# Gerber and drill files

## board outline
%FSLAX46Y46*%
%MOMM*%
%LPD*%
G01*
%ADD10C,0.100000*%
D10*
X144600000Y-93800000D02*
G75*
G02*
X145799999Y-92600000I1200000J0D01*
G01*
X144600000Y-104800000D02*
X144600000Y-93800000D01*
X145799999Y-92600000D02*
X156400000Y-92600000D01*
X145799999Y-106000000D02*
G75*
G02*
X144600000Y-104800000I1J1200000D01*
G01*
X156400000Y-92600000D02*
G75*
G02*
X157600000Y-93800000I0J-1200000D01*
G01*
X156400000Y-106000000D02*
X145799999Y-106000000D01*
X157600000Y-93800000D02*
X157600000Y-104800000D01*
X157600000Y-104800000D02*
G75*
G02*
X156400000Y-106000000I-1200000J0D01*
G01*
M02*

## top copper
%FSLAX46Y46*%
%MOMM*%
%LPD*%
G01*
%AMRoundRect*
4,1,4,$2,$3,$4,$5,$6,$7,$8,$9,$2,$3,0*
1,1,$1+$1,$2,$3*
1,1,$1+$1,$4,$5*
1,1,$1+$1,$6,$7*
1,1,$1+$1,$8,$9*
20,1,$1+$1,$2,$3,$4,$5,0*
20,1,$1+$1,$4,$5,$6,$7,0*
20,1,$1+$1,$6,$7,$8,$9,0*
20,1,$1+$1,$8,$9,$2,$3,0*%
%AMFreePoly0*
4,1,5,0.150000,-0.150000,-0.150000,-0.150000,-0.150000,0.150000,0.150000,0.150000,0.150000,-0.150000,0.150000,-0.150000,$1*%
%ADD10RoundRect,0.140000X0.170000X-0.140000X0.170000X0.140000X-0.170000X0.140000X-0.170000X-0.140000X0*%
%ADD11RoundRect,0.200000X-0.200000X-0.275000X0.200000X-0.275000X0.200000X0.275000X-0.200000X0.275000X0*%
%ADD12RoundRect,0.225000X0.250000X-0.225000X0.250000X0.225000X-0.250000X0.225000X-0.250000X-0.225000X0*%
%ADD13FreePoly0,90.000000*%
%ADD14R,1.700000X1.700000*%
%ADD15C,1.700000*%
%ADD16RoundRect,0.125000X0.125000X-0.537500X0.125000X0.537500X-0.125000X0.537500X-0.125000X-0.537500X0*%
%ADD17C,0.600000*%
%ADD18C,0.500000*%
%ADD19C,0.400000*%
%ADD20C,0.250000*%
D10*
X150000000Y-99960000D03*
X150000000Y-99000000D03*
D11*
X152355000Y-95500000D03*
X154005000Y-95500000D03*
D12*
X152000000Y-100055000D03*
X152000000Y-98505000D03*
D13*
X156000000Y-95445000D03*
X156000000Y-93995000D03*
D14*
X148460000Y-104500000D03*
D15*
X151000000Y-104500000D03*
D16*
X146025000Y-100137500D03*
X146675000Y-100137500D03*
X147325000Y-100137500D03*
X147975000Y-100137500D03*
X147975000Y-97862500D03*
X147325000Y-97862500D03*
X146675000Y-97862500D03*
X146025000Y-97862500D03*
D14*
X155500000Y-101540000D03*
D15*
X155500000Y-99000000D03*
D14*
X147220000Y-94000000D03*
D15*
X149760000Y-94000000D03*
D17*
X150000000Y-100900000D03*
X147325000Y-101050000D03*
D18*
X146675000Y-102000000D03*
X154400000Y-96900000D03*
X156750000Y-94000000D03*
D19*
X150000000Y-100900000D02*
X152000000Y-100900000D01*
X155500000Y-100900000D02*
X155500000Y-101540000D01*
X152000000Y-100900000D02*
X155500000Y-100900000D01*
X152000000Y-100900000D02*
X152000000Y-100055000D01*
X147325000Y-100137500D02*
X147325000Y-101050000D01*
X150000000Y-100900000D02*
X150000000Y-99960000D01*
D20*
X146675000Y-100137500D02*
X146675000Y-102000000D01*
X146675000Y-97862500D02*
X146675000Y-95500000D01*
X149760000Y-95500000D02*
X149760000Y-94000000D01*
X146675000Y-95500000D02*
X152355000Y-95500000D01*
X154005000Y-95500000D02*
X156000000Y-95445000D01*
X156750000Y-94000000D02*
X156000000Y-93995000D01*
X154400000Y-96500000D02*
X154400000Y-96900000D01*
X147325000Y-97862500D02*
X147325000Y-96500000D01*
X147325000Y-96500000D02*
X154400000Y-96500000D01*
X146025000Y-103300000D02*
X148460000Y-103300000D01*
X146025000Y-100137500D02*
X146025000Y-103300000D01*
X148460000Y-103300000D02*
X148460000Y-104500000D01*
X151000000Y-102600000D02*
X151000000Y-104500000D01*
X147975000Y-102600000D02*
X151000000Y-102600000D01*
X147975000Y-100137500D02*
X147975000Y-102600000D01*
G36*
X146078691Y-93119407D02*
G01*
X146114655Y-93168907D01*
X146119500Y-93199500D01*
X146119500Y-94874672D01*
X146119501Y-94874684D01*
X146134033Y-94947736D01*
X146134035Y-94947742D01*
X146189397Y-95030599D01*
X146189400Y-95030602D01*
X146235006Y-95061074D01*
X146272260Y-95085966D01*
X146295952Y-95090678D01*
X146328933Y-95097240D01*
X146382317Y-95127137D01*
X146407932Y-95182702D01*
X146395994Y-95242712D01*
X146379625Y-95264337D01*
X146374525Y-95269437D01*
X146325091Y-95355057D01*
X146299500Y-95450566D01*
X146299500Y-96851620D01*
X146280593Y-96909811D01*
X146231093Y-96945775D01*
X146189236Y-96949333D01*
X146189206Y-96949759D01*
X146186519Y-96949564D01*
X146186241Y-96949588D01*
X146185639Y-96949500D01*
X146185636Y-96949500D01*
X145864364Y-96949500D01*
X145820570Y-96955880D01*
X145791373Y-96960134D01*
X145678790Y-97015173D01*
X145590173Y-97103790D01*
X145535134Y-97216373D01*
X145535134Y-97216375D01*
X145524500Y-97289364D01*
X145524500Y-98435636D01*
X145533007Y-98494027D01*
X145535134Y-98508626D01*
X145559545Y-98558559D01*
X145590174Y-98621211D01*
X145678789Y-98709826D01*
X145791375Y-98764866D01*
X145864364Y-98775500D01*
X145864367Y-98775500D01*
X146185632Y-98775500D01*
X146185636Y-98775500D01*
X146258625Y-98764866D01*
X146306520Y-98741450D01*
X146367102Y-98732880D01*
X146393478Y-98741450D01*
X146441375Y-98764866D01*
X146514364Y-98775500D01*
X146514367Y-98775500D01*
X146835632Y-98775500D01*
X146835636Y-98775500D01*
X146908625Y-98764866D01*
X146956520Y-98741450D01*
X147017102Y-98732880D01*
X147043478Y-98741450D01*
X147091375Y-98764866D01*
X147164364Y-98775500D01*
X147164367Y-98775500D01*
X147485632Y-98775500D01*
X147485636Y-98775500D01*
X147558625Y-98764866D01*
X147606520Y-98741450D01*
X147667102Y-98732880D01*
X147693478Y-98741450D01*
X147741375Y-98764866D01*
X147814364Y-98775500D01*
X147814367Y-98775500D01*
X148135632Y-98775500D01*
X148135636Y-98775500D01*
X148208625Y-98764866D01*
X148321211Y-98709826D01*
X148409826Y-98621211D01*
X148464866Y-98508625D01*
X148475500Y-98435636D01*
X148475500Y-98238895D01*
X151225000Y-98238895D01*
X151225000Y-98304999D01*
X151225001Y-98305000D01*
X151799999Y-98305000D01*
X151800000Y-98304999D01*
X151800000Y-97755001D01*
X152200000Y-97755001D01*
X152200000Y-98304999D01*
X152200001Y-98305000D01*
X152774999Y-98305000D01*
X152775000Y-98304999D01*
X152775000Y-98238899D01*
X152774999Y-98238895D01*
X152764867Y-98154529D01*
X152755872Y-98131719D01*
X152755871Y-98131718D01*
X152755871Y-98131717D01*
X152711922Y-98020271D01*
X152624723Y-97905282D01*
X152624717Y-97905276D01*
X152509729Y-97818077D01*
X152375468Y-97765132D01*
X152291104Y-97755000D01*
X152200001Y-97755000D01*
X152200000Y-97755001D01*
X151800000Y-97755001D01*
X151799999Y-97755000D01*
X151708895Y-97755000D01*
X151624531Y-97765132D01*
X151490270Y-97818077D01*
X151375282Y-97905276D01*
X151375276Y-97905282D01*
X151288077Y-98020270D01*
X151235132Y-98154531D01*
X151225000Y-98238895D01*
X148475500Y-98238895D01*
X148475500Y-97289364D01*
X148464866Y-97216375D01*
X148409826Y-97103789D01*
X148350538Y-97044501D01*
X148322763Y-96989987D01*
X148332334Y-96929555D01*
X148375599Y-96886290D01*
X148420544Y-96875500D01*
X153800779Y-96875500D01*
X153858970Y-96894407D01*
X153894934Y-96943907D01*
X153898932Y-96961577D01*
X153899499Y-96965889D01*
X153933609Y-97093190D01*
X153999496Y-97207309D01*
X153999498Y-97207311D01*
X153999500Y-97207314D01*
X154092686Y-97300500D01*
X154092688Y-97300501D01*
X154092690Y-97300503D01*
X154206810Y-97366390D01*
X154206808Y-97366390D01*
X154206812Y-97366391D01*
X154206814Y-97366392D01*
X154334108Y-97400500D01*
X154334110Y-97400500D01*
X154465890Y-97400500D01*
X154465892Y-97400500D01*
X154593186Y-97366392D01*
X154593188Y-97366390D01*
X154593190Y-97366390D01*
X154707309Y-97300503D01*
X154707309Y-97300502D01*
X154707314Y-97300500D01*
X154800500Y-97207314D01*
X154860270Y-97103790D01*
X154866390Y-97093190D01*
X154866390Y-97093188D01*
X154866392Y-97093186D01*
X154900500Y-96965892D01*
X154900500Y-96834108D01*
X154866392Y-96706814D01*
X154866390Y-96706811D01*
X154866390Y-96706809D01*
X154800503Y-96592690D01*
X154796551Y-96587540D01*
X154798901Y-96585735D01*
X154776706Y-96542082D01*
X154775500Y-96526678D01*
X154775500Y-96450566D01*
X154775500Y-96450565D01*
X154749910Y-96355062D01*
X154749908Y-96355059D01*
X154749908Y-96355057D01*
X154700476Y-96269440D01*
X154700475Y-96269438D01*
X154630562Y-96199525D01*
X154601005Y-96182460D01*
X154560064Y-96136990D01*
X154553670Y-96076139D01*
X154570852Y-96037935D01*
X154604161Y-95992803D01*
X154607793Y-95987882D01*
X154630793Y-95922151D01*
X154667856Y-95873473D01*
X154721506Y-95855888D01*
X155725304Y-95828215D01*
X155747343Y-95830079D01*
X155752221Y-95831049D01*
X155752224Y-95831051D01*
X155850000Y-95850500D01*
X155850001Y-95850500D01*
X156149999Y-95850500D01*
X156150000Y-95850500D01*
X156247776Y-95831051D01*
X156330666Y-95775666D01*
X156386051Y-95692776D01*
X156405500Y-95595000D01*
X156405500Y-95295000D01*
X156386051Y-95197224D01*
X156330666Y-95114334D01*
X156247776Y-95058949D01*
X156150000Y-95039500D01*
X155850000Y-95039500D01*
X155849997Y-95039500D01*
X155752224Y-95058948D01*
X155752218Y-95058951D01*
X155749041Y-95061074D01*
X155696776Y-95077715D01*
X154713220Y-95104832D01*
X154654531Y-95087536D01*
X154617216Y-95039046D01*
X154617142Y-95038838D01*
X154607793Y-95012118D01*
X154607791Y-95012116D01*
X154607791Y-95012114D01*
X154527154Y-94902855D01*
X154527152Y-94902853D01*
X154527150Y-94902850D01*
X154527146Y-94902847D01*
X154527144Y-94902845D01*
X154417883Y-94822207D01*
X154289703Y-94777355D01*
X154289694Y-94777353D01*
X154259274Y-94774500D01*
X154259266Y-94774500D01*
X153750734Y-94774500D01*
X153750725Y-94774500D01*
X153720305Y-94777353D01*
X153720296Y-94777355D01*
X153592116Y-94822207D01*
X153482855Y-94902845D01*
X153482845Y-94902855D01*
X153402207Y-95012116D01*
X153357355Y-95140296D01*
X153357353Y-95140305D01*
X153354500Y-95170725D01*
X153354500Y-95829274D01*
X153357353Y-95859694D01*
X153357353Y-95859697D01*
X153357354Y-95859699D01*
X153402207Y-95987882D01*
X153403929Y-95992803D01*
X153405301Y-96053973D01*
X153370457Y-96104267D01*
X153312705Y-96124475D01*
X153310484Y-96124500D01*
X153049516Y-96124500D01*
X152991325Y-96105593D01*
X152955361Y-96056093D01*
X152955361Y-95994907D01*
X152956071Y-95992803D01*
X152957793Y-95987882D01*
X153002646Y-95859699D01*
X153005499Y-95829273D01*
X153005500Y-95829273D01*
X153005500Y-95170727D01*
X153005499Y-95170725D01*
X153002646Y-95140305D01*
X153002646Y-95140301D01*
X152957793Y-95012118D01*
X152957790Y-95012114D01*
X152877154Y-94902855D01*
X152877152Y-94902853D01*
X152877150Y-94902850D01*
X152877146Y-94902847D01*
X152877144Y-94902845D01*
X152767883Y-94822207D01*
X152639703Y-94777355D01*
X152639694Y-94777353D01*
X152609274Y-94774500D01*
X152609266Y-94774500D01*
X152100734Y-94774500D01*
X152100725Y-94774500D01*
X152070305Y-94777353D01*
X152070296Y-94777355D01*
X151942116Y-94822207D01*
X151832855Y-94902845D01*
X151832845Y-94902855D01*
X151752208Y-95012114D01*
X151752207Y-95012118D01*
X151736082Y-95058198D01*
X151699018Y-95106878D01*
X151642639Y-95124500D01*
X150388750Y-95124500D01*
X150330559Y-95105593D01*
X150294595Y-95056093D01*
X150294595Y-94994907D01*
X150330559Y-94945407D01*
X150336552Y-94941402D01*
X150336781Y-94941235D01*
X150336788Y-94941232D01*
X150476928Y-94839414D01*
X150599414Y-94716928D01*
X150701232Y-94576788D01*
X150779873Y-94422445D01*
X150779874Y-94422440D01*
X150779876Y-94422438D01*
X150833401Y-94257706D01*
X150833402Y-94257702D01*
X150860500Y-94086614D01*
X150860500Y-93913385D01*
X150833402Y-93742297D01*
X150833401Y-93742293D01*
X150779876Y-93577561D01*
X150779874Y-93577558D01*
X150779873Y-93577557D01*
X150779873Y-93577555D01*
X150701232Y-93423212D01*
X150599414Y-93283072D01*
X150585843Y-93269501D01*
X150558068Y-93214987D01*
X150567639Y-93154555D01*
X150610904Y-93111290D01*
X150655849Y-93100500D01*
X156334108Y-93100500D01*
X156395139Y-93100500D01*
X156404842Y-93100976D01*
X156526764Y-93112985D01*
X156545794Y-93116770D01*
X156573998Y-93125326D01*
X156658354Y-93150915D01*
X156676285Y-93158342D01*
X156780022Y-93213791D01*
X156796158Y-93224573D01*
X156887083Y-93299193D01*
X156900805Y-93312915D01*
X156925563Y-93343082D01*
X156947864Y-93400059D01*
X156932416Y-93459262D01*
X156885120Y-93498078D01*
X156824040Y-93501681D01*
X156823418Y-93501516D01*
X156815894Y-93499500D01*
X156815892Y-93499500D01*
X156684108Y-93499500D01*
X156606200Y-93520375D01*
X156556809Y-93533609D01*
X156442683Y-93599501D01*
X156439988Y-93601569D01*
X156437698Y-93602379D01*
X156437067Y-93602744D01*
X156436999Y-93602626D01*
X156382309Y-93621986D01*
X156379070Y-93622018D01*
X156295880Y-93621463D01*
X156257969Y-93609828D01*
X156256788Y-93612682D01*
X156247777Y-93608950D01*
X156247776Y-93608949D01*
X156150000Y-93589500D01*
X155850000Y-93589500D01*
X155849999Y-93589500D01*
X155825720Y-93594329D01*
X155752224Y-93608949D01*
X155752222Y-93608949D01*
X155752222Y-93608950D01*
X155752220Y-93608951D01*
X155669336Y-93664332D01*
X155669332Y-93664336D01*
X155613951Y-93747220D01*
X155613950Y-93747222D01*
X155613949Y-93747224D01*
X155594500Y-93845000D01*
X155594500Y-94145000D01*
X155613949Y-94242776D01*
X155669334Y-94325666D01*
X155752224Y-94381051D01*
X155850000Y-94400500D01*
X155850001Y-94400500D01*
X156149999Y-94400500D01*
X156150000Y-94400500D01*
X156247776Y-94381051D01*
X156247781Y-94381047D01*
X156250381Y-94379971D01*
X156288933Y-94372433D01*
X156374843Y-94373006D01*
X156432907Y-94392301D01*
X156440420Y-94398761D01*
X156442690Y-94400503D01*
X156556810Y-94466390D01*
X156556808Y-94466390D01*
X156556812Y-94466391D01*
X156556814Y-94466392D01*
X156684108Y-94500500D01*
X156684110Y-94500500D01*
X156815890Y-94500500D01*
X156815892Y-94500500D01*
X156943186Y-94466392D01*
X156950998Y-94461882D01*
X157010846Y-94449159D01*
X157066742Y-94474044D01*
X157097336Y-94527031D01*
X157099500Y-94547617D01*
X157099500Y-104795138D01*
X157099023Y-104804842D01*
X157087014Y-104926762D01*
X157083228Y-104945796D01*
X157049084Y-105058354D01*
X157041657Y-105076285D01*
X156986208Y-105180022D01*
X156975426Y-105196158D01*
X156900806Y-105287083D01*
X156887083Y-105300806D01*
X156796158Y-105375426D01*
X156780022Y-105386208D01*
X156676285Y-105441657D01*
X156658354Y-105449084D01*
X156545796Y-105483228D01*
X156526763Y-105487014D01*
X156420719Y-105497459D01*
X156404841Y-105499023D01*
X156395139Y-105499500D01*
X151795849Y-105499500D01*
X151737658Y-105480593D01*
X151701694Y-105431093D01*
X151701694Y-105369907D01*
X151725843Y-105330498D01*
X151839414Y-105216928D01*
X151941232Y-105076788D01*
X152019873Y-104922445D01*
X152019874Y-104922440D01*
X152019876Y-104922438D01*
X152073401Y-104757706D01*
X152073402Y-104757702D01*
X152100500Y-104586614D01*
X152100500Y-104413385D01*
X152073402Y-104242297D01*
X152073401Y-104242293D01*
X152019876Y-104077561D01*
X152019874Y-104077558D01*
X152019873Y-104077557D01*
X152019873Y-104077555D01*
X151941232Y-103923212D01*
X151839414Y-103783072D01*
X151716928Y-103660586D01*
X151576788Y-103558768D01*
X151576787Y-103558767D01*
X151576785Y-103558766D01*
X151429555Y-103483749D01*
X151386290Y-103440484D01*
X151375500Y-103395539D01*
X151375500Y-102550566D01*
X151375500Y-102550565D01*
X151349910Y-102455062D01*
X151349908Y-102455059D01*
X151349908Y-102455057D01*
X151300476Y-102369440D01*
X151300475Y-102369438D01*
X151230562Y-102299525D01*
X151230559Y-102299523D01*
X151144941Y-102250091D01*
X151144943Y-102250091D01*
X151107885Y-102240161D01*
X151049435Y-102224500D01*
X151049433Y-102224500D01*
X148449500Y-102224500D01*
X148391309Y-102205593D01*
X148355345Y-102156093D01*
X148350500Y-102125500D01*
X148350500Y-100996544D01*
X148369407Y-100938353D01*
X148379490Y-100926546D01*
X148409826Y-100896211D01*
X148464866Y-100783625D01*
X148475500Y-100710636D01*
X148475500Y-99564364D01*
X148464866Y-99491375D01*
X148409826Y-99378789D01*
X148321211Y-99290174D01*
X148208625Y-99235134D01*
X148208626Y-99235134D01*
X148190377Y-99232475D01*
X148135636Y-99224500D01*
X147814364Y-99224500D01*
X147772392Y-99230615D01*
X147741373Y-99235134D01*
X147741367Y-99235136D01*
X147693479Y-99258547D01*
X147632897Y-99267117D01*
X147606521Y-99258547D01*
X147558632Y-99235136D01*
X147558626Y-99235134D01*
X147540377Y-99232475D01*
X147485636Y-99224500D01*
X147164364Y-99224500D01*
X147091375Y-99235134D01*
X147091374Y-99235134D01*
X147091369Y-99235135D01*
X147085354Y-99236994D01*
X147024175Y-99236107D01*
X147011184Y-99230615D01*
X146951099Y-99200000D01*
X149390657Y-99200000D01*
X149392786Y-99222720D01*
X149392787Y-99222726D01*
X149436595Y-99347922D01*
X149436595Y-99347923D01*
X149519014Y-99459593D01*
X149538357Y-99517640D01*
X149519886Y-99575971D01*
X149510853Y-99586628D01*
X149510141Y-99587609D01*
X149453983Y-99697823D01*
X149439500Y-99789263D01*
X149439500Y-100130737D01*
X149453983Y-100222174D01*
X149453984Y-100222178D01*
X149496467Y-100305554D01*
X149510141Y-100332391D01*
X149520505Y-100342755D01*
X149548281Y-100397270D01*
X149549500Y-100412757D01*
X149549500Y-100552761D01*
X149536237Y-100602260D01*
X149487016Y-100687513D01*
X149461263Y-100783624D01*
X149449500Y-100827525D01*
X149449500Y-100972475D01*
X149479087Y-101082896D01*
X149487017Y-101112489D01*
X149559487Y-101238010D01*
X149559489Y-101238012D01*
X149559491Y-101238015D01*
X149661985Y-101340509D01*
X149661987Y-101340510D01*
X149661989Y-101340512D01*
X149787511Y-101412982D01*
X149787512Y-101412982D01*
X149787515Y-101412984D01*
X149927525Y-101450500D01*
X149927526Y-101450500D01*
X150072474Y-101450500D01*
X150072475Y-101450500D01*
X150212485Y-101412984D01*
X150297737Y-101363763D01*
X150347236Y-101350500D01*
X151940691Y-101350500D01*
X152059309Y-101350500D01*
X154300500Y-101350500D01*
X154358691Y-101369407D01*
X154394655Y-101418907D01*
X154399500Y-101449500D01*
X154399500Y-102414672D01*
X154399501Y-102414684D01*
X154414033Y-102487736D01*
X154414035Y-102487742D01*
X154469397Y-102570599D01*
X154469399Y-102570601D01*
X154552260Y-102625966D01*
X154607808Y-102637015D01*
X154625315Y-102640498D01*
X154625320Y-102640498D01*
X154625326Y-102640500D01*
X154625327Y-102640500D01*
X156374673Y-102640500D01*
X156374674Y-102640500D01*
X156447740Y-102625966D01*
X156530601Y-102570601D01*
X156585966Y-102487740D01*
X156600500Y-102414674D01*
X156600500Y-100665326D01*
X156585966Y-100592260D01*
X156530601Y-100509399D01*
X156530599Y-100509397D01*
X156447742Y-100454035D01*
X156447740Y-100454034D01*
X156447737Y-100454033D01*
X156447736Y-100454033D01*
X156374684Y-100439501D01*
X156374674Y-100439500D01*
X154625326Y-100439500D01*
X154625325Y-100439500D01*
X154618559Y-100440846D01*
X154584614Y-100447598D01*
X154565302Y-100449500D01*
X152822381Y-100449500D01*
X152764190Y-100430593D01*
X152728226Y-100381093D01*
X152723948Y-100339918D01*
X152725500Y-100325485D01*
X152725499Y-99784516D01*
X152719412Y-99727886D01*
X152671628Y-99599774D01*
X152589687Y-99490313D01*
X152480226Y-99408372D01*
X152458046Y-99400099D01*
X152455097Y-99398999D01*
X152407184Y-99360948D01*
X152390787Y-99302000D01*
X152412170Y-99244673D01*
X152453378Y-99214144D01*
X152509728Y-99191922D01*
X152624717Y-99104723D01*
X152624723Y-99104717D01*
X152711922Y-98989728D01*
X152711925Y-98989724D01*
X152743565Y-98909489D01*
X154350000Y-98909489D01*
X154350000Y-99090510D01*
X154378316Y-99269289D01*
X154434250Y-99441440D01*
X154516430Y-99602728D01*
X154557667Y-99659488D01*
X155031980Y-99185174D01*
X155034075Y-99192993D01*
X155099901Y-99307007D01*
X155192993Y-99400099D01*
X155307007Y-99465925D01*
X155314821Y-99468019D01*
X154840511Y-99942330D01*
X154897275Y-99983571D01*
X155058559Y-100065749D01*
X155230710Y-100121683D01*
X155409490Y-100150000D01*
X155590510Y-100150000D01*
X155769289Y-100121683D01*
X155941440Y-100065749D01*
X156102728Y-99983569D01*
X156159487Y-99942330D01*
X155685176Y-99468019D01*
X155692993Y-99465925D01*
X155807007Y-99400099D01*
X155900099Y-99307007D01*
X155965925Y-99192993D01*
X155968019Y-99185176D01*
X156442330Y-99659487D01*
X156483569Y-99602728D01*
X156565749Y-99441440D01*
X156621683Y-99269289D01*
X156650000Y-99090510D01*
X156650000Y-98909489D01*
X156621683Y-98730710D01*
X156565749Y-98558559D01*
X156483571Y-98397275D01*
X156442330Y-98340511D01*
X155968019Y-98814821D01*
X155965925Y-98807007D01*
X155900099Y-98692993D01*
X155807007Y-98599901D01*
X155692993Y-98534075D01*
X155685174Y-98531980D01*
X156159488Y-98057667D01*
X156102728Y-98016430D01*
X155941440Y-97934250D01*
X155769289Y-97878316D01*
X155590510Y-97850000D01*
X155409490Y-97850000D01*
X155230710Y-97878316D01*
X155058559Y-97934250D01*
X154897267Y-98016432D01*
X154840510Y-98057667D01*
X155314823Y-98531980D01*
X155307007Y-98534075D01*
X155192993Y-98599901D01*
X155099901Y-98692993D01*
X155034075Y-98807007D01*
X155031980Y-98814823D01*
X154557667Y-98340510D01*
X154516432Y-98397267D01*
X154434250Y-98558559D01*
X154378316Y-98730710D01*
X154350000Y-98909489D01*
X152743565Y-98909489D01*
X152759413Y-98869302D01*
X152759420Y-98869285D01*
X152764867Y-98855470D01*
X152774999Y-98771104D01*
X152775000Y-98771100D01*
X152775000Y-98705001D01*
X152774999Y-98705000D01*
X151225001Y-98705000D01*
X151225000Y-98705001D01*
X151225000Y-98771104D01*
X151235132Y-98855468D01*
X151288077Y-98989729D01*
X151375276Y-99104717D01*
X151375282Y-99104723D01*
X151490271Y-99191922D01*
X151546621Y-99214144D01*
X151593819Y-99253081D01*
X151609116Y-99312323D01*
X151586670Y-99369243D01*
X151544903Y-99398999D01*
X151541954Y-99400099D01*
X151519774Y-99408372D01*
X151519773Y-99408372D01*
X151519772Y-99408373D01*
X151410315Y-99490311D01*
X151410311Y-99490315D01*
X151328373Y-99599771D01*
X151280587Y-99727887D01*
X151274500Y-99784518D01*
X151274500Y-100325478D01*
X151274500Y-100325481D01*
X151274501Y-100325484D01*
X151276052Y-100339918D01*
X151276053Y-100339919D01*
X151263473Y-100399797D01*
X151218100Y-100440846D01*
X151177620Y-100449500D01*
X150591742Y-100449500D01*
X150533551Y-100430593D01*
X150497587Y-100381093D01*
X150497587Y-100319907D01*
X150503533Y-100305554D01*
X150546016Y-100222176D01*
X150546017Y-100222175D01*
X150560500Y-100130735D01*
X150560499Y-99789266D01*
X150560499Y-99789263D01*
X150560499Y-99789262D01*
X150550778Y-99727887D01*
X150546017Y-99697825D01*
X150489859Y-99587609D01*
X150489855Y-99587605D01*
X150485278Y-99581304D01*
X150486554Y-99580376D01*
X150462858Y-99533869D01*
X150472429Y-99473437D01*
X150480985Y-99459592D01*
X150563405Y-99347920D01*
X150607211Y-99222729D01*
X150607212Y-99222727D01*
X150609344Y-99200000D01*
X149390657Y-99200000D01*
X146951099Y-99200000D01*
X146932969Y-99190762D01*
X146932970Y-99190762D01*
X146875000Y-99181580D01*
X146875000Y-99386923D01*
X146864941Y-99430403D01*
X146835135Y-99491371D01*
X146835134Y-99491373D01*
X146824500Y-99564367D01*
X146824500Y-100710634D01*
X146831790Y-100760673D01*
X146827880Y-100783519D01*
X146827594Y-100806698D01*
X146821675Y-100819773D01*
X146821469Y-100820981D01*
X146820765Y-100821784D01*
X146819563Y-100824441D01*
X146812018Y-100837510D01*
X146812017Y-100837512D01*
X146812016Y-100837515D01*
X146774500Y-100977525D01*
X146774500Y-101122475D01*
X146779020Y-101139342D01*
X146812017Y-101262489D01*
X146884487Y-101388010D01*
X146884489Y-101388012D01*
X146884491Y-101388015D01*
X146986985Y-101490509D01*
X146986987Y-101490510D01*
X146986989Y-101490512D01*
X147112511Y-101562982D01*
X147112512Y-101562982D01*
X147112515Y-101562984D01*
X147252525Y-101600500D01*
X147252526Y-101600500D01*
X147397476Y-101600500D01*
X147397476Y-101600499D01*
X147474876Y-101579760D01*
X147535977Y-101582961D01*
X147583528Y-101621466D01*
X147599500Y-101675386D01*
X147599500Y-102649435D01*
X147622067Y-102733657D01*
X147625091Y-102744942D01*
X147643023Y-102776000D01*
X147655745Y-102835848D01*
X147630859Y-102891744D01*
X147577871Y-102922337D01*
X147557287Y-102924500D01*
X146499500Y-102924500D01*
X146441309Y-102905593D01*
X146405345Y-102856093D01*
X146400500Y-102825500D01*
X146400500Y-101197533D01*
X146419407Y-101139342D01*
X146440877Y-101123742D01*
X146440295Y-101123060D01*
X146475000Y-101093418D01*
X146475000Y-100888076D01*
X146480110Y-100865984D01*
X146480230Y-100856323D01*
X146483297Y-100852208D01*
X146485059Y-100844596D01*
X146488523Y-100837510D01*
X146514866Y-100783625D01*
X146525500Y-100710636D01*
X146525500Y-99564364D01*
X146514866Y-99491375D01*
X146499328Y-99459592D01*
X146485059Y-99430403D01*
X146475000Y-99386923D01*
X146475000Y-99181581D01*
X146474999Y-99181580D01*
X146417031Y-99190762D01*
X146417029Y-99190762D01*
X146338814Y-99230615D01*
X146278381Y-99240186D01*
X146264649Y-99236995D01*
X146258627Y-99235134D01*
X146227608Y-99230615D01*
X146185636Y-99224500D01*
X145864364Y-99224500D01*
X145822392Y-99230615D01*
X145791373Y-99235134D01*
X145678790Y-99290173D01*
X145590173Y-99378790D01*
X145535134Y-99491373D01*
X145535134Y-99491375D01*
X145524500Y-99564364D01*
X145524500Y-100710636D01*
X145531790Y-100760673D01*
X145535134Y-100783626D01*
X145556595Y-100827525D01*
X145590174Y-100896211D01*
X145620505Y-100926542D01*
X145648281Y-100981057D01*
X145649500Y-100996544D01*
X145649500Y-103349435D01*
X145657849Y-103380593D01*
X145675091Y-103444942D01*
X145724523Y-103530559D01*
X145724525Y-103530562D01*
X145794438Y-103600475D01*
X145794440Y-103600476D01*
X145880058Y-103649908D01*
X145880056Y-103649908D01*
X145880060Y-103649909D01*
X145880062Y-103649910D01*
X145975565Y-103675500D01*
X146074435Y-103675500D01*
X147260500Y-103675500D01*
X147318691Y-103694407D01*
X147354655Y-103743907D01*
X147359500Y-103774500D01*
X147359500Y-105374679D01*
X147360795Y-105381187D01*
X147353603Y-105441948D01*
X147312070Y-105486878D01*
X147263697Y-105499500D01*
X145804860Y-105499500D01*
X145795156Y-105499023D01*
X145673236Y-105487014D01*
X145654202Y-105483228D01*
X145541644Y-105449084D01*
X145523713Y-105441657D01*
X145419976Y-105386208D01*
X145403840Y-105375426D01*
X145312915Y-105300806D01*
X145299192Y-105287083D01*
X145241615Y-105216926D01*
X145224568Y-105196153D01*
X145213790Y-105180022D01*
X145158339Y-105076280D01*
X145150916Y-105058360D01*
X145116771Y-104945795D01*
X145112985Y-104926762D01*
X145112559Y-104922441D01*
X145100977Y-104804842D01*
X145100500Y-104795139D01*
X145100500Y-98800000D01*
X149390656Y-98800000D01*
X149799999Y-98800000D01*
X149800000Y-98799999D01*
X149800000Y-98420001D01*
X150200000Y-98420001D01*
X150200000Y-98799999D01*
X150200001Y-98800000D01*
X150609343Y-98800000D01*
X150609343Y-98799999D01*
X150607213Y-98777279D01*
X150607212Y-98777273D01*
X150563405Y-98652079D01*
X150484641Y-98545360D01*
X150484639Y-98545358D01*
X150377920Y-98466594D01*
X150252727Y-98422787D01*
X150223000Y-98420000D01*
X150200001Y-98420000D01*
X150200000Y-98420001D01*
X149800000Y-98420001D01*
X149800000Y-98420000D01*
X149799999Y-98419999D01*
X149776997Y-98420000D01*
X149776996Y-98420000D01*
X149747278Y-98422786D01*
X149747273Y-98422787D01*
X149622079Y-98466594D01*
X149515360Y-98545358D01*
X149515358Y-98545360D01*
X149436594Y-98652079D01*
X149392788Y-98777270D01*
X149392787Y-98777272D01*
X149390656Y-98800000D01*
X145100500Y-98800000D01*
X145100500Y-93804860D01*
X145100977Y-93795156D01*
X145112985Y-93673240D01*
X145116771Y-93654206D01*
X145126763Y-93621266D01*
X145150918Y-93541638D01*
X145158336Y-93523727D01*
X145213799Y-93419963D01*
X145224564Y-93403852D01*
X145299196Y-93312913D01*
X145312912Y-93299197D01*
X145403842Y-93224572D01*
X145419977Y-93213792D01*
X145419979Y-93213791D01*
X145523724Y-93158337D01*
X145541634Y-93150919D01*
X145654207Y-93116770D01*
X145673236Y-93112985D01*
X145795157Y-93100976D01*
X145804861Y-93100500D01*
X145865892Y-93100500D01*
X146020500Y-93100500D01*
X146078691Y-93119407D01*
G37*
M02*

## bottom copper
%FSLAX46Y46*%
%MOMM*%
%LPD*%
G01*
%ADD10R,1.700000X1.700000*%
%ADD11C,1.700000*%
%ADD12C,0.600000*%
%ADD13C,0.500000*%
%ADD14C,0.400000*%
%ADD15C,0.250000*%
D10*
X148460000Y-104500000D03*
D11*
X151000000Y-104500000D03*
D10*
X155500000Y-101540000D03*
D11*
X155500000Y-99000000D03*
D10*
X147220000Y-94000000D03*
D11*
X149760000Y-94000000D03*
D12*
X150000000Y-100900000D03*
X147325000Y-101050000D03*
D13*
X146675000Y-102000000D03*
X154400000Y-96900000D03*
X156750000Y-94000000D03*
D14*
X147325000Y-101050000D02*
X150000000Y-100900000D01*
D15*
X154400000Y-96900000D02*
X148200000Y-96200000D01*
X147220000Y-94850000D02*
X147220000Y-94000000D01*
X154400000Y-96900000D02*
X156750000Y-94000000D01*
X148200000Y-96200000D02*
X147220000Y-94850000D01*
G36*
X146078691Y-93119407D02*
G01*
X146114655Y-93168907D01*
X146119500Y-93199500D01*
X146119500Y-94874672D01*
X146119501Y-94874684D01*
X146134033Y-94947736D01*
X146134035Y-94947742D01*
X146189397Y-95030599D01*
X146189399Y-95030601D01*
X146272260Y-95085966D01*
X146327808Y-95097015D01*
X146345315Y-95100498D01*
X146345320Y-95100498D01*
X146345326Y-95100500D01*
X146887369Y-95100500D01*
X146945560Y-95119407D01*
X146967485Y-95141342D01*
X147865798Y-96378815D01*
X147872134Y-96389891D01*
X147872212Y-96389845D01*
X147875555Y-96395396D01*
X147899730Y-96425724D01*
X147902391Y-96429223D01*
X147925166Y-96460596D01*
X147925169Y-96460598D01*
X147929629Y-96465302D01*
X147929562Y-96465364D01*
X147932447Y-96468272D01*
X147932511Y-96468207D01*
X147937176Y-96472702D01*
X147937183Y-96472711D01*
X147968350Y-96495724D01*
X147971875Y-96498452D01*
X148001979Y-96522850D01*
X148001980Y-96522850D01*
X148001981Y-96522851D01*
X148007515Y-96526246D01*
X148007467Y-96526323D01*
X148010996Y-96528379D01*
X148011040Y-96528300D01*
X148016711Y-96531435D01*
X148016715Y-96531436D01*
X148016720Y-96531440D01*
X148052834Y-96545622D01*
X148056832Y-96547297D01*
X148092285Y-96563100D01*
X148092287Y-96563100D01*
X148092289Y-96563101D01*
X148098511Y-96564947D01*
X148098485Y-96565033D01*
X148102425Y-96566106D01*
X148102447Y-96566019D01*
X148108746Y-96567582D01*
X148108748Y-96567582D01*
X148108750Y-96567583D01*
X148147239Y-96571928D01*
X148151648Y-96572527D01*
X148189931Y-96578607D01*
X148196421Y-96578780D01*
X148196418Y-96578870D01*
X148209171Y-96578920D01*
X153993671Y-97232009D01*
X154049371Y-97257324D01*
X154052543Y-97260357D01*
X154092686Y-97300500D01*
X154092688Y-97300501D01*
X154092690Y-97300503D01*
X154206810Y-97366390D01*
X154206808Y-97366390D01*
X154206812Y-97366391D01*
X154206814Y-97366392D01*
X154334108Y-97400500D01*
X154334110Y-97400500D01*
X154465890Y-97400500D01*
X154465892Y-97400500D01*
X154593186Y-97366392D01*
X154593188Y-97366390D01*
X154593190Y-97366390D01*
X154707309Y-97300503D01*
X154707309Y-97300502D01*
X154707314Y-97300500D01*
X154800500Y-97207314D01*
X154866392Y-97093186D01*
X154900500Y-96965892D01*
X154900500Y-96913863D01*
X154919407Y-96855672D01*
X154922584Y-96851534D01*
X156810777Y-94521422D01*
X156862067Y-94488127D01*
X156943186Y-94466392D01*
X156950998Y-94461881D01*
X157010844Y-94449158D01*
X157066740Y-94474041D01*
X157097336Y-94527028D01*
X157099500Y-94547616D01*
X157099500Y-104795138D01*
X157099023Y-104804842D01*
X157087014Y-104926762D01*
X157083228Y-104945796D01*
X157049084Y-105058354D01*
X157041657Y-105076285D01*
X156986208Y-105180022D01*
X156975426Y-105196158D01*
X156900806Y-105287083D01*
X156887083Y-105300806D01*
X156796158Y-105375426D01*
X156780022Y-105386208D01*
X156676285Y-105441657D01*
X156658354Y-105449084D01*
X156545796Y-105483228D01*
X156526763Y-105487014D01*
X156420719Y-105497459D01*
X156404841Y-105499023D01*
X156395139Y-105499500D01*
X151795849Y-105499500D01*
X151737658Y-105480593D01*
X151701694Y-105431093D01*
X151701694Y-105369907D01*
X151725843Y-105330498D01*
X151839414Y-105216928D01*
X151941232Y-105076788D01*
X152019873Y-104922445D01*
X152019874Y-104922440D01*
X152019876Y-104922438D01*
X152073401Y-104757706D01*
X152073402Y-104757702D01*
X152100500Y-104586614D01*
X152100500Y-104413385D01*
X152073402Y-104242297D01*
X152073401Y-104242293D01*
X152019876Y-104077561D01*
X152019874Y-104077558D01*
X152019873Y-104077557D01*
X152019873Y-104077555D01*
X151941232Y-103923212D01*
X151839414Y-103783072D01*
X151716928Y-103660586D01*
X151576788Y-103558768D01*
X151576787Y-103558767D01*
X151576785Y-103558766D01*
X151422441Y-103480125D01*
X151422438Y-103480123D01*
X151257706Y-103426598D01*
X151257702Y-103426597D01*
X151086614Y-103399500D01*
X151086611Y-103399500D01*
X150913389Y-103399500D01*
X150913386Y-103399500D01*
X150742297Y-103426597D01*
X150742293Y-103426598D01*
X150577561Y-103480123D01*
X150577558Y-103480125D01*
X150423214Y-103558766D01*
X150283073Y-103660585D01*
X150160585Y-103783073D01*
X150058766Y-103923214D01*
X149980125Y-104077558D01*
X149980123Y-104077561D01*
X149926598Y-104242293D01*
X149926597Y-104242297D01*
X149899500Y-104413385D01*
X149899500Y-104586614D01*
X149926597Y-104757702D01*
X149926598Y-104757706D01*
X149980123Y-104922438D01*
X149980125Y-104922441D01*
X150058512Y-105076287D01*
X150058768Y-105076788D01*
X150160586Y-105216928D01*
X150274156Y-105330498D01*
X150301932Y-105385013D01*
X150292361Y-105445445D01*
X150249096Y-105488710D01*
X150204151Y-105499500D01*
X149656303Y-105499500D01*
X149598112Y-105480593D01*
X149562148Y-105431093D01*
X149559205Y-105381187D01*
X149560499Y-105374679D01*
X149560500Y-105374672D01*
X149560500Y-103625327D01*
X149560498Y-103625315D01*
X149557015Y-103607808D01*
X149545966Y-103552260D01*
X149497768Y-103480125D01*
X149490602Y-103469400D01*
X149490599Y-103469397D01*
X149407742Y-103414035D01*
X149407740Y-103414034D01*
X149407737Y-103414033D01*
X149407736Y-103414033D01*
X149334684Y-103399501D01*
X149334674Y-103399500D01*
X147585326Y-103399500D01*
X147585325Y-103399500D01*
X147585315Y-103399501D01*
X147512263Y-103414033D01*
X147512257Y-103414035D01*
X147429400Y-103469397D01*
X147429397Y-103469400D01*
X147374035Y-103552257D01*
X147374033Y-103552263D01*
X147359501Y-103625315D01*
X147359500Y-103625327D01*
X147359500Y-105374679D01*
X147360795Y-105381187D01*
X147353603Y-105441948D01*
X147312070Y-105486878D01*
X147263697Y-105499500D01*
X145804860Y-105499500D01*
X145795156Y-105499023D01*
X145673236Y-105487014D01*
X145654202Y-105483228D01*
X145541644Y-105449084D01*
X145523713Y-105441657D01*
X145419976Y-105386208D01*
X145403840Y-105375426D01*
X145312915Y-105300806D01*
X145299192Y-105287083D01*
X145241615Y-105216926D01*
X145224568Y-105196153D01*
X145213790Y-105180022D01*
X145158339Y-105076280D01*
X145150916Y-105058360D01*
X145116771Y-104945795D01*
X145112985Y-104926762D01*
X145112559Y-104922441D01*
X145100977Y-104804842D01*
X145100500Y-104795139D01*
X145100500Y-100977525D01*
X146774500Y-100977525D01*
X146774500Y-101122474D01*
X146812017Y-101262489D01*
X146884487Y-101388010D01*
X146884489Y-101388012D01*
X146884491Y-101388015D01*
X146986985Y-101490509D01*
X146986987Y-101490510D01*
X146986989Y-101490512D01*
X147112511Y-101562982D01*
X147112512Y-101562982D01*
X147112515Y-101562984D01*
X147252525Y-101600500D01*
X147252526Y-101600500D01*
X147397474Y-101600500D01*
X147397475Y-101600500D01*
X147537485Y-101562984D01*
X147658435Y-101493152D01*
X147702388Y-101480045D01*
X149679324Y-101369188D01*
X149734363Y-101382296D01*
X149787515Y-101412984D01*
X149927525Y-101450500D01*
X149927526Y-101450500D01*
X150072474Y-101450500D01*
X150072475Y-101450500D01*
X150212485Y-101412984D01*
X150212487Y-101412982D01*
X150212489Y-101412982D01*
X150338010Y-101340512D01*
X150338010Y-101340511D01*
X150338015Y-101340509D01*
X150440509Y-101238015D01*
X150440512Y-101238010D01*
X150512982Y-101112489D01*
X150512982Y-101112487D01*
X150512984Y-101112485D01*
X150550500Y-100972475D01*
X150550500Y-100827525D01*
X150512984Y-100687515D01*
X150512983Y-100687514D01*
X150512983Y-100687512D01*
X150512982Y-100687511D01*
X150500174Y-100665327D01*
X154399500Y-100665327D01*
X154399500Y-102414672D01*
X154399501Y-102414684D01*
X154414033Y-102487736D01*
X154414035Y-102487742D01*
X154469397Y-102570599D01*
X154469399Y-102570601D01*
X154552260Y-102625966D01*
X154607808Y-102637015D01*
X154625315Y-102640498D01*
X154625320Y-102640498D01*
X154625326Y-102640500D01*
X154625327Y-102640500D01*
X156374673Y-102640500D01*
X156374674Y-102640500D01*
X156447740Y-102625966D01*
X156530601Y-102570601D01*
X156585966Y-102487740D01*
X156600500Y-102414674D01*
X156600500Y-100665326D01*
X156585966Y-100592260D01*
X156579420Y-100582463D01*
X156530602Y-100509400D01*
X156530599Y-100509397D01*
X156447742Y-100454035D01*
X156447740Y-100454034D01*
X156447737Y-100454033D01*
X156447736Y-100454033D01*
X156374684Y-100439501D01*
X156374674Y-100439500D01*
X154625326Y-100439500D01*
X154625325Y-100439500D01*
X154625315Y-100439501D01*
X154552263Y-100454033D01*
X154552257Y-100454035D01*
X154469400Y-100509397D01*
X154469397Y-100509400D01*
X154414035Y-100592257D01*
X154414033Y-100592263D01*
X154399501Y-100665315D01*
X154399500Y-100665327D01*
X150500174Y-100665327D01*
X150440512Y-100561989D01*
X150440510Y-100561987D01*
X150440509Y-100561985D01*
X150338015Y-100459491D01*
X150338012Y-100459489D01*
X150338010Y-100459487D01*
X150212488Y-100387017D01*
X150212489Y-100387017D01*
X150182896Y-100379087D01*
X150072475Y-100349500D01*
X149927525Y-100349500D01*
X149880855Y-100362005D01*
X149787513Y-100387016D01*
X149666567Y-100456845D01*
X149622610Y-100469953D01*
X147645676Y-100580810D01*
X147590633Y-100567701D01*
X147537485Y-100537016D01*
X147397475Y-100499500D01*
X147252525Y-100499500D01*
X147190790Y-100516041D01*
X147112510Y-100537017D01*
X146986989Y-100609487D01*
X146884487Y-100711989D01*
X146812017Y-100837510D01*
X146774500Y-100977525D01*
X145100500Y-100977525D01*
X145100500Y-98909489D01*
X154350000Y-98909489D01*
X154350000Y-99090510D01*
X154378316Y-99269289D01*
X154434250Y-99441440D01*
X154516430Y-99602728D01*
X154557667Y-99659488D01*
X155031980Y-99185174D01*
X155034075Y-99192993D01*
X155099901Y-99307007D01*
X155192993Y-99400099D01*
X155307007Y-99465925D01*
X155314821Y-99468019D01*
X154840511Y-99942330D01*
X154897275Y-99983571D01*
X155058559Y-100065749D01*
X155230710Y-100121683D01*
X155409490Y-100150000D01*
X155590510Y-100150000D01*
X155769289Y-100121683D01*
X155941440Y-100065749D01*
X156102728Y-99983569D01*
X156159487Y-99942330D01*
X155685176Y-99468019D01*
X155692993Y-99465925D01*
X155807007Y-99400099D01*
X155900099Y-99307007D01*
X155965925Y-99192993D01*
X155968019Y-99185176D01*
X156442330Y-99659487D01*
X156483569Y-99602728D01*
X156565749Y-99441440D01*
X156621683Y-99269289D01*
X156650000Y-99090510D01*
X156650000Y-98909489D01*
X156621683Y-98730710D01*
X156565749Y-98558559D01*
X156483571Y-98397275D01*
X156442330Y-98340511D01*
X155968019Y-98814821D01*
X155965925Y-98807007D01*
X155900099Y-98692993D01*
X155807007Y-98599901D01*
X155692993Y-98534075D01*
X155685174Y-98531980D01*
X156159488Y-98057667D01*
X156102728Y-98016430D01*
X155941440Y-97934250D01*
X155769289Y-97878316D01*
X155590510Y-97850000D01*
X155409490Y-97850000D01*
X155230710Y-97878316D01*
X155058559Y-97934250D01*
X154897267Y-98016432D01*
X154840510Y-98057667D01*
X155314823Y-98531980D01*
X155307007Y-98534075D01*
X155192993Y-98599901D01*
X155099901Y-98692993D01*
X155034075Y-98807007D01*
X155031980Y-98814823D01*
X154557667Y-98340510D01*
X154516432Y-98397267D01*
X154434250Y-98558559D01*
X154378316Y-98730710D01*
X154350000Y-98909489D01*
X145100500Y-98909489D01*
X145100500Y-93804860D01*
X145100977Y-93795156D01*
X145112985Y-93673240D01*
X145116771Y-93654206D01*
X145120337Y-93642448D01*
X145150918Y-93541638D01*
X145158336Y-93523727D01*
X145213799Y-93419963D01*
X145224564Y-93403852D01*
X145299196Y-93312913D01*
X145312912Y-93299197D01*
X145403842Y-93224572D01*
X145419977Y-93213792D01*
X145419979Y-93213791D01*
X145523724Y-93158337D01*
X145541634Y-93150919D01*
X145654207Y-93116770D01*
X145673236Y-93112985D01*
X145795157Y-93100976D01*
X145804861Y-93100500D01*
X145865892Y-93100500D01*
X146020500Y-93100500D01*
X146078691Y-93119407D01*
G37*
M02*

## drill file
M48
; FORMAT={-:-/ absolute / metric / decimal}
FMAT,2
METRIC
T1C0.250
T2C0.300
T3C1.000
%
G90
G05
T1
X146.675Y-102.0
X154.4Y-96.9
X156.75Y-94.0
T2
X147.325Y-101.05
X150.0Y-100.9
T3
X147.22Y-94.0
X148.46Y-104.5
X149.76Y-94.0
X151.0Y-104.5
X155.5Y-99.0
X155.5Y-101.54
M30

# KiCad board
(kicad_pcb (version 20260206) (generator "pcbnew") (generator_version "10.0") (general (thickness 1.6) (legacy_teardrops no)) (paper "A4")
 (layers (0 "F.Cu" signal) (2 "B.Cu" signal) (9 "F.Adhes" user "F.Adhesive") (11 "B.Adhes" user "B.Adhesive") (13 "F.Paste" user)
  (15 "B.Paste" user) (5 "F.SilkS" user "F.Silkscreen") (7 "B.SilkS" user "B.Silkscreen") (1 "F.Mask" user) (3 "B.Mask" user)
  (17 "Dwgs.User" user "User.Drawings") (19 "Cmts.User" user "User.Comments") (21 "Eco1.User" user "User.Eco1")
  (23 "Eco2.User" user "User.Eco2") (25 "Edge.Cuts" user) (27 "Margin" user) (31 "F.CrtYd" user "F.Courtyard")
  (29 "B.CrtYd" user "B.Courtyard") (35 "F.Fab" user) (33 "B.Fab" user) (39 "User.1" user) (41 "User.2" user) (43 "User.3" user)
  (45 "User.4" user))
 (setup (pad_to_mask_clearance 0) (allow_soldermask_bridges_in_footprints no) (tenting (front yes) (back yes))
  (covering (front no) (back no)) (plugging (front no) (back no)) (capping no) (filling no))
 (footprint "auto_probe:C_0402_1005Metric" (layer "F.Cu") (at 150 99.48 90)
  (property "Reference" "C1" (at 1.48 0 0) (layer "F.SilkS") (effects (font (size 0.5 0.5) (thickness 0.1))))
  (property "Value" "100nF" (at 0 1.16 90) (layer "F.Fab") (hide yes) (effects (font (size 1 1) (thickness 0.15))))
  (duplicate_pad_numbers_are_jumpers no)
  (pad "1" smd roundrect (at -0.48 0 90) (size 0.56 0.62) (layers "F.Cu" "F.Mask" "F.Paste") (roundrect_rratio 0.25) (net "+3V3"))
  (pad "2" smd roundrect (at 0.48 0 90) (size 0.56 0.62) (layers "F.Cu" "F.Mask" "F.Paste") (roundrect_rratio 0.25) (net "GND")))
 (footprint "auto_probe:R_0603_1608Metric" (layer "F.Cu") (at 153.18 95.5)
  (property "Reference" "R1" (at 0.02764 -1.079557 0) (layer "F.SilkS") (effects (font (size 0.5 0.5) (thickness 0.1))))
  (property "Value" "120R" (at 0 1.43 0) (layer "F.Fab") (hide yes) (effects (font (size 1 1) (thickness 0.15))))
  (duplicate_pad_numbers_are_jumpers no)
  (pad "1" smd roundrect (at -0.825 0) (size 0.8 0.95) (layers "F.Cu" "F.Mask" "F.Paste") (roundrect_rratio 0.25) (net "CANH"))
  (pad "2" smd roundrect (at 0.825 0) (size 0.8 0.95) (layers "F.Cu" "F.Mask" "F.Paste") (roundrect_rratio 0.25) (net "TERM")))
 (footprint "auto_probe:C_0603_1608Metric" (layer "F.Cu") (at 152 99.28 90)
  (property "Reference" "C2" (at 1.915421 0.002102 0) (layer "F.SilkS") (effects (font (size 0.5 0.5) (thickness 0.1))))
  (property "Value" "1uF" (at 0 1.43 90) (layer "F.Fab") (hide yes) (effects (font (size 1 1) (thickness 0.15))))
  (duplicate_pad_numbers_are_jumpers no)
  (pad "1" smd roundrect (at -0.775 0 90) (size 0.9 0.95) (layers "F.Cu" "F.Mask" "F.Paste") (roundrect_rratio 0.25) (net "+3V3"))
  (pad "2" smd roundrect (at 0.775 0 90) (size 0.9 0.95) (layers "F.Cu" "F.Mask" "F.Paste") (roundrect_rratio 0.25) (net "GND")))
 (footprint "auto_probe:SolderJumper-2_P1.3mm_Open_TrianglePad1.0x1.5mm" (layer "F.Cu") (at 156 94.72 90)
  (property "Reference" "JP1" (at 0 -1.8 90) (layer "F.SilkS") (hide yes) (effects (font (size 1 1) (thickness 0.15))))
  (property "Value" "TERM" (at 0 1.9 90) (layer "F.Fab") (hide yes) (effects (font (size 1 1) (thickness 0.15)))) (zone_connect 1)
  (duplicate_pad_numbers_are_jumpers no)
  (pad "1" smd custom (at -0.725 0 90) (size 0.3 0.3) (layers "F.Cu" "F.Mask") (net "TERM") (zone_connect 2) (thermal_bridge_angle 45)
   (options (clearance outline) (anchor rect)) (primitives))
  (pad "2" smd custom (at 0.725 0 90) (size 0.3 0.3) (layers "F.Cu" "F.Mask") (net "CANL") (zone_connect 2) (thermal_bridge_angle 45)
   (options (clearance outline) (anchor rect)) (primitives)))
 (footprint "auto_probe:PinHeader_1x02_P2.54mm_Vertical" (layer "F.Cu") (at 148.46 104.5 90)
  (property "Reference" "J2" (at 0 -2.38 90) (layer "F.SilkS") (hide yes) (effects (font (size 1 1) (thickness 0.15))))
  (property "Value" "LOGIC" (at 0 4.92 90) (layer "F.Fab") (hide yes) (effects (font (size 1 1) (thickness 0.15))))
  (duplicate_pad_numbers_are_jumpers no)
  (pad "1" thru_hole rect (at 0 0 90) (size 1.7 1.7) (drill 1) (layers "*.Cu" "*.Mask") (remove_unused_layers no) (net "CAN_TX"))
  (pad "2" thru_hole circle (at 0 2.54 90) (size 1.7 1.7) (drill 1) (layers "*.Cu" "*.Mask") (remove_unused_layers no) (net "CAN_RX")))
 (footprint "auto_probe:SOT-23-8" (layer "F.Cu") (at 147 99 90)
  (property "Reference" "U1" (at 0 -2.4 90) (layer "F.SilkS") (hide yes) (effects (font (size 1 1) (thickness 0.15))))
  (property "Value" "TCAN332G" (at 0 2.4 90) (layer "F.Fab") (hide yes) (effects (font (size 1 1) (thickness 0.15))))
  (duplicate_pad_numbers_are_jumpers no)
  (pad "1" smd roundrect (at -1.1375 -0.975 90) (size 1.325 0.5) (layers "F.Cu" "F.Mask" "F.Paste") (roundrect_rratio 0.25) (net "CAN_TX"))
  (pad "2" smd roundrect (at -1.1375 -0.325 90) (size 1.325 0.5) (layers "F.Cu" "F.Mask" "F.Paste") (roundrect_rratio 0.25) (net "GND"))
  (pad "3" smd roundrect (at -1.1375 0.325 90) (size 1.325 0.5) (layers "F.Cu" "F.Mask" "F.Paste") (roundrect_rratio 0.25) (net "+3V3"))
  (pad "4" smd roundrect (at -1.1375 0.975 90) (size 1.325 0.5) (layers "F.Cu" "F.Mask" "F.Paste") (roundrect_rratio 0.25) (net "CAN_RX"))
  (pad "5" smd roundrect (at 1.1375 0.975 90) (size 1.325 0.5) (layers "F.Cu" "F.Mask" "F.Paste") (roundrect_rratio 0.25))
  (pad "6" smd roundrect (at 1.1375 0.325 90) (size 1.325 0.5) (layers "F.Cu" "F.Mask" "F.Paste") (roundrect_rratio 0.25) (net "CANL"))
  (pad "7" smd roundrect (at 1.1375 -0.325 90) (size 1.325 0.5) (layers "F.Cu" "F.Mask" "F.Paste") (roundrect_rratio 0.25) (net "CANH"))
  (pad "8" smd roundrect (at 1.1375 -0.975 90) (size 1.325 0.5) (layers "F.Cu" "F.Mask" "F.Paste") (roundrect_rratio 0.25)))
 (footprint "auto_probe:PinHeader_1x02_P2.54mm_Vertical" (layer "F.Cu") (at 155.5 101.54 180)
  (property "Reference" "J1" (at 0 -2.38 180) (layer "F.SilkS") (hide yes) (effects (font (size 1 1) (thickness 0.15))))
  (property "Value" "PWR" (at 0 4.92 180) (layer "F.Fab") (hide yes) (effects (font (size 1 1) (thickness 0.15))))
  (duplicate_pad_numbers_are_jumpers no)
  (pad "1" thru_hole rect (at 0 0 180) (size 1.7 1.7) (drill 1) (layers "*.Cu" "*.Mask") (remove_unused_layers no) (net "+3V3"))
  (pad "2" thru_hole circle (at 0 2.54 180) (size 1.7 1.7) (drill 1) (layers "*.Cu" "*.Mask") (remove_unused_layers no) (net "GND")))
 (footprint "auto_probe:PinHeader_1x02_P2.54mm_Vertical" (layer "F.Cu") (at 147.22 94 90)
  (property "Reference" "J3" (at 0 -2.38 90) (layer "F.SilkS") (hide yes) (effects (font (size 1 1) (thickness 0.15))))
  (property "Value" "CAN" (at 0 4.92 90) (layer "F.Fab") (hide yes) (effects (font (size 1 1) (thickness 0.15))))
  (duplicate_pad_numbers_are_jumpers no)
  (pad "1" thru_hole rect (at 0 0 90) (size 1.7 1.7) (drill 1) (layers "*.Cu" "*.Mask") (remove_unused_layers no) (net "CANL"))
  (pad "2" thru_hole circle (at 0 2.54 90) (size 1.7 1.7) (drill 1) (layers "*.Cu" "*.Mask") (remove_unused_layers no) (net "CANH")))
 (gr_arc (start 144.6 93.8) (mid 144.951472 92.951473) (end 145.799999 92.6) (stroke (width 0.1) (type default)) (layer "Edge.Cuts"))
 (gr_line (start 144.6 104.8) (end 144.6 93.8) (stroke (width 0.1) (type default)) (layer "Edge.Cuts"))
 (gr_line (start 145.799999 92.6) (end 156.4 92.6) (stroke (width 0.1) (type default)) (layer "Edge.Cuts"))
 (gr_arc (start 145.799999 106) (mid 144.951471 105.648528) (end 144.6 104.8) (stroke (width 0.1) (type default)) (layer "Edge.Cuts"))
 (gr_arc (start 156.4 92.6) (mid 157.248528 92.951472) (end 157.6 93.8) (stroke (width 0.1) (type default)) (layer "Edge.Cuts"))
 (gr_line (start 156.4 106) (end 145.799999 106) (stroke (width 0.1) (type default)) (layer "Edge.Cuts"))
 (gr_line (start 157.6 93.8) (end 157.6 104.8) (stroke (width 0.1) (type default)) (layer "Edge.Cuts"))
 (gr_arc (start 157.6 104.8) (mid 157.248528 105.648528) (end 156.4 106) (stroke (width 0.1) (type default)) (layer "Edge.Cuts"))
 (segment (start 150 100.9) (end 152 100.9) (width 0.4) (layer "F.Cu") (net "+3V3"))
 (segment (start 155.5 100.9) (end 155.5 101.54) (width 0.4) (layer "F.Cu") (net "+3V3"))
 (segment (start 152 100.9) (end 155.5 100.9) (width 0.4) (layer "F.Cu") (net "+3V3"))
 (segment (start 152 100.9) (end 152 100.055) (width 0.4) (layer "F.Cu") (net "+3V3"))
 (segment (start 147.325 100.1375) (end 147.325 101.05) (width 0.4) (layer "F.Cu") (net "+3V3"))
 (segment (start 150 100.9) (end 150 99.96) (width 0.4) (layer "F.Cu") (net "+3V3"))
 (via (at 150 100.9) (size 0.6) (drill 0.3) (layers "F.Cu" "B.Cu") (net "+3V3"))
 (via (at 147.325 101.05) (size 0.6) (drill 0.3) (layers "F.Cu" "B.Cu") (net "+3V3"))
 (segment (start 147.325 101.05) (end 150 100.9) (width 0.4) (layer "B.Cu") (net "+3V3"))
 (segment (start 146.675 100.1375) (end 146.675 102) (width 0.25) (layer "F.Cu") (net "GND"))
 (via (at 146.675 102) (size 0.5) (drill 0.25) (layers "F.Cu" "B.Cu") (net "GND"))
 (segment (start 146.675 97.8625) (end 146.675 95.5) (width 0.25) (layer "F.Cu") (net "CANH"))
 (segment (start 149.76 95.5) (end 149.76 94) (width 0.25) (layer "F.Cu") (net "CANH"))
 (segment (start 146.675 95.5) (end 152.355 95.5) (width 0.25) (layer "F.Cu") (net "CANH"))
 (segment (start 154.005 95.5) (end 156 95.445) (width 0.25) (layer "F.Cu") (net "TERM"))
 (segment (start 156.75 94) (end 156 93.995) (width 0.25) (layer "F.Cu") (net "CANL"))
 (segment (start 154.4 96.5) (end 154.4 96.9) (width 0.25) (layer "F.Cu") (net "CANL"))
 (segment (start 147.325 97.8625) (end 147.325 96.5) (width 0.25) (layer "F.Cu") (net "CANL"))
 (segment (start 147.325 96.5) (end 154.4 96.5) (width 0.25) (layer "F.Cu") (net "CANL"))
 (via (at 154.4 96.9) (size 0.5) (drill 0.25) (layers "F.Cu" "B.Cu") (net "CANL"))
 (via (at 156.75 94) (size 0.5) (drill 0.25) (layers "F.Cu" "B.Cu") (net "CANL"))
 (segment (start 154.4 96.9) (end 148.2 96.2) (width 0.25) (layer "B.Cu") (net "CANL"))
 (segment (start 147.22 94.85) (end 147.22 94) (width 0.25) (layer "B.Cu") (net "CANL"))
 (segment (start 154.4 96.9) (end 156.75 94) (width 0.25) (layer "B.Cu") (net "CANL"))
 (segment (start 148.2 96.2) (end 147.22 94.85) (width 0.25) (layer "B.Cu") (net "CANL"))
 (segment (start 146.025 103.3) (end 148.46 103.3) (width 0.25) (layer "F.Cu") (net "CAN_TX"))
 (segment (start 146.025 100.1375) (end 146.025 103.3) (width 0.25) (layer "F.Cu") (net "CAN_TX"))
 (segment (start 148.46 103.3) (end 148.46 104.5) (width 0.25) (layer "F.Cu") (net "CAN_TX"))
 (segment (start 151 102.6) (end 151 104.5) (width 0.25) (layer "F.Cu") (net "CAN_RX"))
 (segment (start 147.975 102.6) (end 151 102.6) (width 0.25) (layer "F.Cu") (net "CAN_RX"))
 (segment (start 147.975 100.1375) (end 147.975 102.6) (width 0.25) (layer "F.Cu") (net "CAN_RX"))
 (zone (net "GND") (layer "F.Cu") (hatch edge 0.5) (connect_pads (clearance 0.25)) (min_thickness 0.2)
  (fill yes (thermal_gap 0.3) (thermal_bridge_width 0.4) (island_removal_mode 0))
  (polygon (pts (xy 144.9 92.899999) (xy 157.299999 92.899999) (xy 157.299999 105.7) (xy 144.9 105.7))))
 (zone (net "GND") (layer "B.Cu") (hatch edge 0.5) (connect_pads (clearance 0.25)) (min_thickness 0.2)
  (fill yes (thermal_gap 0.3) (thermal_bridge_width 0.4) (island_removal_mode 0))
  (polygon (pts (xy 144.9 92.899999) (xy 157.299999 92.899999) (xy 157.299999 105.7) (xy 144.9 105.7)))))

